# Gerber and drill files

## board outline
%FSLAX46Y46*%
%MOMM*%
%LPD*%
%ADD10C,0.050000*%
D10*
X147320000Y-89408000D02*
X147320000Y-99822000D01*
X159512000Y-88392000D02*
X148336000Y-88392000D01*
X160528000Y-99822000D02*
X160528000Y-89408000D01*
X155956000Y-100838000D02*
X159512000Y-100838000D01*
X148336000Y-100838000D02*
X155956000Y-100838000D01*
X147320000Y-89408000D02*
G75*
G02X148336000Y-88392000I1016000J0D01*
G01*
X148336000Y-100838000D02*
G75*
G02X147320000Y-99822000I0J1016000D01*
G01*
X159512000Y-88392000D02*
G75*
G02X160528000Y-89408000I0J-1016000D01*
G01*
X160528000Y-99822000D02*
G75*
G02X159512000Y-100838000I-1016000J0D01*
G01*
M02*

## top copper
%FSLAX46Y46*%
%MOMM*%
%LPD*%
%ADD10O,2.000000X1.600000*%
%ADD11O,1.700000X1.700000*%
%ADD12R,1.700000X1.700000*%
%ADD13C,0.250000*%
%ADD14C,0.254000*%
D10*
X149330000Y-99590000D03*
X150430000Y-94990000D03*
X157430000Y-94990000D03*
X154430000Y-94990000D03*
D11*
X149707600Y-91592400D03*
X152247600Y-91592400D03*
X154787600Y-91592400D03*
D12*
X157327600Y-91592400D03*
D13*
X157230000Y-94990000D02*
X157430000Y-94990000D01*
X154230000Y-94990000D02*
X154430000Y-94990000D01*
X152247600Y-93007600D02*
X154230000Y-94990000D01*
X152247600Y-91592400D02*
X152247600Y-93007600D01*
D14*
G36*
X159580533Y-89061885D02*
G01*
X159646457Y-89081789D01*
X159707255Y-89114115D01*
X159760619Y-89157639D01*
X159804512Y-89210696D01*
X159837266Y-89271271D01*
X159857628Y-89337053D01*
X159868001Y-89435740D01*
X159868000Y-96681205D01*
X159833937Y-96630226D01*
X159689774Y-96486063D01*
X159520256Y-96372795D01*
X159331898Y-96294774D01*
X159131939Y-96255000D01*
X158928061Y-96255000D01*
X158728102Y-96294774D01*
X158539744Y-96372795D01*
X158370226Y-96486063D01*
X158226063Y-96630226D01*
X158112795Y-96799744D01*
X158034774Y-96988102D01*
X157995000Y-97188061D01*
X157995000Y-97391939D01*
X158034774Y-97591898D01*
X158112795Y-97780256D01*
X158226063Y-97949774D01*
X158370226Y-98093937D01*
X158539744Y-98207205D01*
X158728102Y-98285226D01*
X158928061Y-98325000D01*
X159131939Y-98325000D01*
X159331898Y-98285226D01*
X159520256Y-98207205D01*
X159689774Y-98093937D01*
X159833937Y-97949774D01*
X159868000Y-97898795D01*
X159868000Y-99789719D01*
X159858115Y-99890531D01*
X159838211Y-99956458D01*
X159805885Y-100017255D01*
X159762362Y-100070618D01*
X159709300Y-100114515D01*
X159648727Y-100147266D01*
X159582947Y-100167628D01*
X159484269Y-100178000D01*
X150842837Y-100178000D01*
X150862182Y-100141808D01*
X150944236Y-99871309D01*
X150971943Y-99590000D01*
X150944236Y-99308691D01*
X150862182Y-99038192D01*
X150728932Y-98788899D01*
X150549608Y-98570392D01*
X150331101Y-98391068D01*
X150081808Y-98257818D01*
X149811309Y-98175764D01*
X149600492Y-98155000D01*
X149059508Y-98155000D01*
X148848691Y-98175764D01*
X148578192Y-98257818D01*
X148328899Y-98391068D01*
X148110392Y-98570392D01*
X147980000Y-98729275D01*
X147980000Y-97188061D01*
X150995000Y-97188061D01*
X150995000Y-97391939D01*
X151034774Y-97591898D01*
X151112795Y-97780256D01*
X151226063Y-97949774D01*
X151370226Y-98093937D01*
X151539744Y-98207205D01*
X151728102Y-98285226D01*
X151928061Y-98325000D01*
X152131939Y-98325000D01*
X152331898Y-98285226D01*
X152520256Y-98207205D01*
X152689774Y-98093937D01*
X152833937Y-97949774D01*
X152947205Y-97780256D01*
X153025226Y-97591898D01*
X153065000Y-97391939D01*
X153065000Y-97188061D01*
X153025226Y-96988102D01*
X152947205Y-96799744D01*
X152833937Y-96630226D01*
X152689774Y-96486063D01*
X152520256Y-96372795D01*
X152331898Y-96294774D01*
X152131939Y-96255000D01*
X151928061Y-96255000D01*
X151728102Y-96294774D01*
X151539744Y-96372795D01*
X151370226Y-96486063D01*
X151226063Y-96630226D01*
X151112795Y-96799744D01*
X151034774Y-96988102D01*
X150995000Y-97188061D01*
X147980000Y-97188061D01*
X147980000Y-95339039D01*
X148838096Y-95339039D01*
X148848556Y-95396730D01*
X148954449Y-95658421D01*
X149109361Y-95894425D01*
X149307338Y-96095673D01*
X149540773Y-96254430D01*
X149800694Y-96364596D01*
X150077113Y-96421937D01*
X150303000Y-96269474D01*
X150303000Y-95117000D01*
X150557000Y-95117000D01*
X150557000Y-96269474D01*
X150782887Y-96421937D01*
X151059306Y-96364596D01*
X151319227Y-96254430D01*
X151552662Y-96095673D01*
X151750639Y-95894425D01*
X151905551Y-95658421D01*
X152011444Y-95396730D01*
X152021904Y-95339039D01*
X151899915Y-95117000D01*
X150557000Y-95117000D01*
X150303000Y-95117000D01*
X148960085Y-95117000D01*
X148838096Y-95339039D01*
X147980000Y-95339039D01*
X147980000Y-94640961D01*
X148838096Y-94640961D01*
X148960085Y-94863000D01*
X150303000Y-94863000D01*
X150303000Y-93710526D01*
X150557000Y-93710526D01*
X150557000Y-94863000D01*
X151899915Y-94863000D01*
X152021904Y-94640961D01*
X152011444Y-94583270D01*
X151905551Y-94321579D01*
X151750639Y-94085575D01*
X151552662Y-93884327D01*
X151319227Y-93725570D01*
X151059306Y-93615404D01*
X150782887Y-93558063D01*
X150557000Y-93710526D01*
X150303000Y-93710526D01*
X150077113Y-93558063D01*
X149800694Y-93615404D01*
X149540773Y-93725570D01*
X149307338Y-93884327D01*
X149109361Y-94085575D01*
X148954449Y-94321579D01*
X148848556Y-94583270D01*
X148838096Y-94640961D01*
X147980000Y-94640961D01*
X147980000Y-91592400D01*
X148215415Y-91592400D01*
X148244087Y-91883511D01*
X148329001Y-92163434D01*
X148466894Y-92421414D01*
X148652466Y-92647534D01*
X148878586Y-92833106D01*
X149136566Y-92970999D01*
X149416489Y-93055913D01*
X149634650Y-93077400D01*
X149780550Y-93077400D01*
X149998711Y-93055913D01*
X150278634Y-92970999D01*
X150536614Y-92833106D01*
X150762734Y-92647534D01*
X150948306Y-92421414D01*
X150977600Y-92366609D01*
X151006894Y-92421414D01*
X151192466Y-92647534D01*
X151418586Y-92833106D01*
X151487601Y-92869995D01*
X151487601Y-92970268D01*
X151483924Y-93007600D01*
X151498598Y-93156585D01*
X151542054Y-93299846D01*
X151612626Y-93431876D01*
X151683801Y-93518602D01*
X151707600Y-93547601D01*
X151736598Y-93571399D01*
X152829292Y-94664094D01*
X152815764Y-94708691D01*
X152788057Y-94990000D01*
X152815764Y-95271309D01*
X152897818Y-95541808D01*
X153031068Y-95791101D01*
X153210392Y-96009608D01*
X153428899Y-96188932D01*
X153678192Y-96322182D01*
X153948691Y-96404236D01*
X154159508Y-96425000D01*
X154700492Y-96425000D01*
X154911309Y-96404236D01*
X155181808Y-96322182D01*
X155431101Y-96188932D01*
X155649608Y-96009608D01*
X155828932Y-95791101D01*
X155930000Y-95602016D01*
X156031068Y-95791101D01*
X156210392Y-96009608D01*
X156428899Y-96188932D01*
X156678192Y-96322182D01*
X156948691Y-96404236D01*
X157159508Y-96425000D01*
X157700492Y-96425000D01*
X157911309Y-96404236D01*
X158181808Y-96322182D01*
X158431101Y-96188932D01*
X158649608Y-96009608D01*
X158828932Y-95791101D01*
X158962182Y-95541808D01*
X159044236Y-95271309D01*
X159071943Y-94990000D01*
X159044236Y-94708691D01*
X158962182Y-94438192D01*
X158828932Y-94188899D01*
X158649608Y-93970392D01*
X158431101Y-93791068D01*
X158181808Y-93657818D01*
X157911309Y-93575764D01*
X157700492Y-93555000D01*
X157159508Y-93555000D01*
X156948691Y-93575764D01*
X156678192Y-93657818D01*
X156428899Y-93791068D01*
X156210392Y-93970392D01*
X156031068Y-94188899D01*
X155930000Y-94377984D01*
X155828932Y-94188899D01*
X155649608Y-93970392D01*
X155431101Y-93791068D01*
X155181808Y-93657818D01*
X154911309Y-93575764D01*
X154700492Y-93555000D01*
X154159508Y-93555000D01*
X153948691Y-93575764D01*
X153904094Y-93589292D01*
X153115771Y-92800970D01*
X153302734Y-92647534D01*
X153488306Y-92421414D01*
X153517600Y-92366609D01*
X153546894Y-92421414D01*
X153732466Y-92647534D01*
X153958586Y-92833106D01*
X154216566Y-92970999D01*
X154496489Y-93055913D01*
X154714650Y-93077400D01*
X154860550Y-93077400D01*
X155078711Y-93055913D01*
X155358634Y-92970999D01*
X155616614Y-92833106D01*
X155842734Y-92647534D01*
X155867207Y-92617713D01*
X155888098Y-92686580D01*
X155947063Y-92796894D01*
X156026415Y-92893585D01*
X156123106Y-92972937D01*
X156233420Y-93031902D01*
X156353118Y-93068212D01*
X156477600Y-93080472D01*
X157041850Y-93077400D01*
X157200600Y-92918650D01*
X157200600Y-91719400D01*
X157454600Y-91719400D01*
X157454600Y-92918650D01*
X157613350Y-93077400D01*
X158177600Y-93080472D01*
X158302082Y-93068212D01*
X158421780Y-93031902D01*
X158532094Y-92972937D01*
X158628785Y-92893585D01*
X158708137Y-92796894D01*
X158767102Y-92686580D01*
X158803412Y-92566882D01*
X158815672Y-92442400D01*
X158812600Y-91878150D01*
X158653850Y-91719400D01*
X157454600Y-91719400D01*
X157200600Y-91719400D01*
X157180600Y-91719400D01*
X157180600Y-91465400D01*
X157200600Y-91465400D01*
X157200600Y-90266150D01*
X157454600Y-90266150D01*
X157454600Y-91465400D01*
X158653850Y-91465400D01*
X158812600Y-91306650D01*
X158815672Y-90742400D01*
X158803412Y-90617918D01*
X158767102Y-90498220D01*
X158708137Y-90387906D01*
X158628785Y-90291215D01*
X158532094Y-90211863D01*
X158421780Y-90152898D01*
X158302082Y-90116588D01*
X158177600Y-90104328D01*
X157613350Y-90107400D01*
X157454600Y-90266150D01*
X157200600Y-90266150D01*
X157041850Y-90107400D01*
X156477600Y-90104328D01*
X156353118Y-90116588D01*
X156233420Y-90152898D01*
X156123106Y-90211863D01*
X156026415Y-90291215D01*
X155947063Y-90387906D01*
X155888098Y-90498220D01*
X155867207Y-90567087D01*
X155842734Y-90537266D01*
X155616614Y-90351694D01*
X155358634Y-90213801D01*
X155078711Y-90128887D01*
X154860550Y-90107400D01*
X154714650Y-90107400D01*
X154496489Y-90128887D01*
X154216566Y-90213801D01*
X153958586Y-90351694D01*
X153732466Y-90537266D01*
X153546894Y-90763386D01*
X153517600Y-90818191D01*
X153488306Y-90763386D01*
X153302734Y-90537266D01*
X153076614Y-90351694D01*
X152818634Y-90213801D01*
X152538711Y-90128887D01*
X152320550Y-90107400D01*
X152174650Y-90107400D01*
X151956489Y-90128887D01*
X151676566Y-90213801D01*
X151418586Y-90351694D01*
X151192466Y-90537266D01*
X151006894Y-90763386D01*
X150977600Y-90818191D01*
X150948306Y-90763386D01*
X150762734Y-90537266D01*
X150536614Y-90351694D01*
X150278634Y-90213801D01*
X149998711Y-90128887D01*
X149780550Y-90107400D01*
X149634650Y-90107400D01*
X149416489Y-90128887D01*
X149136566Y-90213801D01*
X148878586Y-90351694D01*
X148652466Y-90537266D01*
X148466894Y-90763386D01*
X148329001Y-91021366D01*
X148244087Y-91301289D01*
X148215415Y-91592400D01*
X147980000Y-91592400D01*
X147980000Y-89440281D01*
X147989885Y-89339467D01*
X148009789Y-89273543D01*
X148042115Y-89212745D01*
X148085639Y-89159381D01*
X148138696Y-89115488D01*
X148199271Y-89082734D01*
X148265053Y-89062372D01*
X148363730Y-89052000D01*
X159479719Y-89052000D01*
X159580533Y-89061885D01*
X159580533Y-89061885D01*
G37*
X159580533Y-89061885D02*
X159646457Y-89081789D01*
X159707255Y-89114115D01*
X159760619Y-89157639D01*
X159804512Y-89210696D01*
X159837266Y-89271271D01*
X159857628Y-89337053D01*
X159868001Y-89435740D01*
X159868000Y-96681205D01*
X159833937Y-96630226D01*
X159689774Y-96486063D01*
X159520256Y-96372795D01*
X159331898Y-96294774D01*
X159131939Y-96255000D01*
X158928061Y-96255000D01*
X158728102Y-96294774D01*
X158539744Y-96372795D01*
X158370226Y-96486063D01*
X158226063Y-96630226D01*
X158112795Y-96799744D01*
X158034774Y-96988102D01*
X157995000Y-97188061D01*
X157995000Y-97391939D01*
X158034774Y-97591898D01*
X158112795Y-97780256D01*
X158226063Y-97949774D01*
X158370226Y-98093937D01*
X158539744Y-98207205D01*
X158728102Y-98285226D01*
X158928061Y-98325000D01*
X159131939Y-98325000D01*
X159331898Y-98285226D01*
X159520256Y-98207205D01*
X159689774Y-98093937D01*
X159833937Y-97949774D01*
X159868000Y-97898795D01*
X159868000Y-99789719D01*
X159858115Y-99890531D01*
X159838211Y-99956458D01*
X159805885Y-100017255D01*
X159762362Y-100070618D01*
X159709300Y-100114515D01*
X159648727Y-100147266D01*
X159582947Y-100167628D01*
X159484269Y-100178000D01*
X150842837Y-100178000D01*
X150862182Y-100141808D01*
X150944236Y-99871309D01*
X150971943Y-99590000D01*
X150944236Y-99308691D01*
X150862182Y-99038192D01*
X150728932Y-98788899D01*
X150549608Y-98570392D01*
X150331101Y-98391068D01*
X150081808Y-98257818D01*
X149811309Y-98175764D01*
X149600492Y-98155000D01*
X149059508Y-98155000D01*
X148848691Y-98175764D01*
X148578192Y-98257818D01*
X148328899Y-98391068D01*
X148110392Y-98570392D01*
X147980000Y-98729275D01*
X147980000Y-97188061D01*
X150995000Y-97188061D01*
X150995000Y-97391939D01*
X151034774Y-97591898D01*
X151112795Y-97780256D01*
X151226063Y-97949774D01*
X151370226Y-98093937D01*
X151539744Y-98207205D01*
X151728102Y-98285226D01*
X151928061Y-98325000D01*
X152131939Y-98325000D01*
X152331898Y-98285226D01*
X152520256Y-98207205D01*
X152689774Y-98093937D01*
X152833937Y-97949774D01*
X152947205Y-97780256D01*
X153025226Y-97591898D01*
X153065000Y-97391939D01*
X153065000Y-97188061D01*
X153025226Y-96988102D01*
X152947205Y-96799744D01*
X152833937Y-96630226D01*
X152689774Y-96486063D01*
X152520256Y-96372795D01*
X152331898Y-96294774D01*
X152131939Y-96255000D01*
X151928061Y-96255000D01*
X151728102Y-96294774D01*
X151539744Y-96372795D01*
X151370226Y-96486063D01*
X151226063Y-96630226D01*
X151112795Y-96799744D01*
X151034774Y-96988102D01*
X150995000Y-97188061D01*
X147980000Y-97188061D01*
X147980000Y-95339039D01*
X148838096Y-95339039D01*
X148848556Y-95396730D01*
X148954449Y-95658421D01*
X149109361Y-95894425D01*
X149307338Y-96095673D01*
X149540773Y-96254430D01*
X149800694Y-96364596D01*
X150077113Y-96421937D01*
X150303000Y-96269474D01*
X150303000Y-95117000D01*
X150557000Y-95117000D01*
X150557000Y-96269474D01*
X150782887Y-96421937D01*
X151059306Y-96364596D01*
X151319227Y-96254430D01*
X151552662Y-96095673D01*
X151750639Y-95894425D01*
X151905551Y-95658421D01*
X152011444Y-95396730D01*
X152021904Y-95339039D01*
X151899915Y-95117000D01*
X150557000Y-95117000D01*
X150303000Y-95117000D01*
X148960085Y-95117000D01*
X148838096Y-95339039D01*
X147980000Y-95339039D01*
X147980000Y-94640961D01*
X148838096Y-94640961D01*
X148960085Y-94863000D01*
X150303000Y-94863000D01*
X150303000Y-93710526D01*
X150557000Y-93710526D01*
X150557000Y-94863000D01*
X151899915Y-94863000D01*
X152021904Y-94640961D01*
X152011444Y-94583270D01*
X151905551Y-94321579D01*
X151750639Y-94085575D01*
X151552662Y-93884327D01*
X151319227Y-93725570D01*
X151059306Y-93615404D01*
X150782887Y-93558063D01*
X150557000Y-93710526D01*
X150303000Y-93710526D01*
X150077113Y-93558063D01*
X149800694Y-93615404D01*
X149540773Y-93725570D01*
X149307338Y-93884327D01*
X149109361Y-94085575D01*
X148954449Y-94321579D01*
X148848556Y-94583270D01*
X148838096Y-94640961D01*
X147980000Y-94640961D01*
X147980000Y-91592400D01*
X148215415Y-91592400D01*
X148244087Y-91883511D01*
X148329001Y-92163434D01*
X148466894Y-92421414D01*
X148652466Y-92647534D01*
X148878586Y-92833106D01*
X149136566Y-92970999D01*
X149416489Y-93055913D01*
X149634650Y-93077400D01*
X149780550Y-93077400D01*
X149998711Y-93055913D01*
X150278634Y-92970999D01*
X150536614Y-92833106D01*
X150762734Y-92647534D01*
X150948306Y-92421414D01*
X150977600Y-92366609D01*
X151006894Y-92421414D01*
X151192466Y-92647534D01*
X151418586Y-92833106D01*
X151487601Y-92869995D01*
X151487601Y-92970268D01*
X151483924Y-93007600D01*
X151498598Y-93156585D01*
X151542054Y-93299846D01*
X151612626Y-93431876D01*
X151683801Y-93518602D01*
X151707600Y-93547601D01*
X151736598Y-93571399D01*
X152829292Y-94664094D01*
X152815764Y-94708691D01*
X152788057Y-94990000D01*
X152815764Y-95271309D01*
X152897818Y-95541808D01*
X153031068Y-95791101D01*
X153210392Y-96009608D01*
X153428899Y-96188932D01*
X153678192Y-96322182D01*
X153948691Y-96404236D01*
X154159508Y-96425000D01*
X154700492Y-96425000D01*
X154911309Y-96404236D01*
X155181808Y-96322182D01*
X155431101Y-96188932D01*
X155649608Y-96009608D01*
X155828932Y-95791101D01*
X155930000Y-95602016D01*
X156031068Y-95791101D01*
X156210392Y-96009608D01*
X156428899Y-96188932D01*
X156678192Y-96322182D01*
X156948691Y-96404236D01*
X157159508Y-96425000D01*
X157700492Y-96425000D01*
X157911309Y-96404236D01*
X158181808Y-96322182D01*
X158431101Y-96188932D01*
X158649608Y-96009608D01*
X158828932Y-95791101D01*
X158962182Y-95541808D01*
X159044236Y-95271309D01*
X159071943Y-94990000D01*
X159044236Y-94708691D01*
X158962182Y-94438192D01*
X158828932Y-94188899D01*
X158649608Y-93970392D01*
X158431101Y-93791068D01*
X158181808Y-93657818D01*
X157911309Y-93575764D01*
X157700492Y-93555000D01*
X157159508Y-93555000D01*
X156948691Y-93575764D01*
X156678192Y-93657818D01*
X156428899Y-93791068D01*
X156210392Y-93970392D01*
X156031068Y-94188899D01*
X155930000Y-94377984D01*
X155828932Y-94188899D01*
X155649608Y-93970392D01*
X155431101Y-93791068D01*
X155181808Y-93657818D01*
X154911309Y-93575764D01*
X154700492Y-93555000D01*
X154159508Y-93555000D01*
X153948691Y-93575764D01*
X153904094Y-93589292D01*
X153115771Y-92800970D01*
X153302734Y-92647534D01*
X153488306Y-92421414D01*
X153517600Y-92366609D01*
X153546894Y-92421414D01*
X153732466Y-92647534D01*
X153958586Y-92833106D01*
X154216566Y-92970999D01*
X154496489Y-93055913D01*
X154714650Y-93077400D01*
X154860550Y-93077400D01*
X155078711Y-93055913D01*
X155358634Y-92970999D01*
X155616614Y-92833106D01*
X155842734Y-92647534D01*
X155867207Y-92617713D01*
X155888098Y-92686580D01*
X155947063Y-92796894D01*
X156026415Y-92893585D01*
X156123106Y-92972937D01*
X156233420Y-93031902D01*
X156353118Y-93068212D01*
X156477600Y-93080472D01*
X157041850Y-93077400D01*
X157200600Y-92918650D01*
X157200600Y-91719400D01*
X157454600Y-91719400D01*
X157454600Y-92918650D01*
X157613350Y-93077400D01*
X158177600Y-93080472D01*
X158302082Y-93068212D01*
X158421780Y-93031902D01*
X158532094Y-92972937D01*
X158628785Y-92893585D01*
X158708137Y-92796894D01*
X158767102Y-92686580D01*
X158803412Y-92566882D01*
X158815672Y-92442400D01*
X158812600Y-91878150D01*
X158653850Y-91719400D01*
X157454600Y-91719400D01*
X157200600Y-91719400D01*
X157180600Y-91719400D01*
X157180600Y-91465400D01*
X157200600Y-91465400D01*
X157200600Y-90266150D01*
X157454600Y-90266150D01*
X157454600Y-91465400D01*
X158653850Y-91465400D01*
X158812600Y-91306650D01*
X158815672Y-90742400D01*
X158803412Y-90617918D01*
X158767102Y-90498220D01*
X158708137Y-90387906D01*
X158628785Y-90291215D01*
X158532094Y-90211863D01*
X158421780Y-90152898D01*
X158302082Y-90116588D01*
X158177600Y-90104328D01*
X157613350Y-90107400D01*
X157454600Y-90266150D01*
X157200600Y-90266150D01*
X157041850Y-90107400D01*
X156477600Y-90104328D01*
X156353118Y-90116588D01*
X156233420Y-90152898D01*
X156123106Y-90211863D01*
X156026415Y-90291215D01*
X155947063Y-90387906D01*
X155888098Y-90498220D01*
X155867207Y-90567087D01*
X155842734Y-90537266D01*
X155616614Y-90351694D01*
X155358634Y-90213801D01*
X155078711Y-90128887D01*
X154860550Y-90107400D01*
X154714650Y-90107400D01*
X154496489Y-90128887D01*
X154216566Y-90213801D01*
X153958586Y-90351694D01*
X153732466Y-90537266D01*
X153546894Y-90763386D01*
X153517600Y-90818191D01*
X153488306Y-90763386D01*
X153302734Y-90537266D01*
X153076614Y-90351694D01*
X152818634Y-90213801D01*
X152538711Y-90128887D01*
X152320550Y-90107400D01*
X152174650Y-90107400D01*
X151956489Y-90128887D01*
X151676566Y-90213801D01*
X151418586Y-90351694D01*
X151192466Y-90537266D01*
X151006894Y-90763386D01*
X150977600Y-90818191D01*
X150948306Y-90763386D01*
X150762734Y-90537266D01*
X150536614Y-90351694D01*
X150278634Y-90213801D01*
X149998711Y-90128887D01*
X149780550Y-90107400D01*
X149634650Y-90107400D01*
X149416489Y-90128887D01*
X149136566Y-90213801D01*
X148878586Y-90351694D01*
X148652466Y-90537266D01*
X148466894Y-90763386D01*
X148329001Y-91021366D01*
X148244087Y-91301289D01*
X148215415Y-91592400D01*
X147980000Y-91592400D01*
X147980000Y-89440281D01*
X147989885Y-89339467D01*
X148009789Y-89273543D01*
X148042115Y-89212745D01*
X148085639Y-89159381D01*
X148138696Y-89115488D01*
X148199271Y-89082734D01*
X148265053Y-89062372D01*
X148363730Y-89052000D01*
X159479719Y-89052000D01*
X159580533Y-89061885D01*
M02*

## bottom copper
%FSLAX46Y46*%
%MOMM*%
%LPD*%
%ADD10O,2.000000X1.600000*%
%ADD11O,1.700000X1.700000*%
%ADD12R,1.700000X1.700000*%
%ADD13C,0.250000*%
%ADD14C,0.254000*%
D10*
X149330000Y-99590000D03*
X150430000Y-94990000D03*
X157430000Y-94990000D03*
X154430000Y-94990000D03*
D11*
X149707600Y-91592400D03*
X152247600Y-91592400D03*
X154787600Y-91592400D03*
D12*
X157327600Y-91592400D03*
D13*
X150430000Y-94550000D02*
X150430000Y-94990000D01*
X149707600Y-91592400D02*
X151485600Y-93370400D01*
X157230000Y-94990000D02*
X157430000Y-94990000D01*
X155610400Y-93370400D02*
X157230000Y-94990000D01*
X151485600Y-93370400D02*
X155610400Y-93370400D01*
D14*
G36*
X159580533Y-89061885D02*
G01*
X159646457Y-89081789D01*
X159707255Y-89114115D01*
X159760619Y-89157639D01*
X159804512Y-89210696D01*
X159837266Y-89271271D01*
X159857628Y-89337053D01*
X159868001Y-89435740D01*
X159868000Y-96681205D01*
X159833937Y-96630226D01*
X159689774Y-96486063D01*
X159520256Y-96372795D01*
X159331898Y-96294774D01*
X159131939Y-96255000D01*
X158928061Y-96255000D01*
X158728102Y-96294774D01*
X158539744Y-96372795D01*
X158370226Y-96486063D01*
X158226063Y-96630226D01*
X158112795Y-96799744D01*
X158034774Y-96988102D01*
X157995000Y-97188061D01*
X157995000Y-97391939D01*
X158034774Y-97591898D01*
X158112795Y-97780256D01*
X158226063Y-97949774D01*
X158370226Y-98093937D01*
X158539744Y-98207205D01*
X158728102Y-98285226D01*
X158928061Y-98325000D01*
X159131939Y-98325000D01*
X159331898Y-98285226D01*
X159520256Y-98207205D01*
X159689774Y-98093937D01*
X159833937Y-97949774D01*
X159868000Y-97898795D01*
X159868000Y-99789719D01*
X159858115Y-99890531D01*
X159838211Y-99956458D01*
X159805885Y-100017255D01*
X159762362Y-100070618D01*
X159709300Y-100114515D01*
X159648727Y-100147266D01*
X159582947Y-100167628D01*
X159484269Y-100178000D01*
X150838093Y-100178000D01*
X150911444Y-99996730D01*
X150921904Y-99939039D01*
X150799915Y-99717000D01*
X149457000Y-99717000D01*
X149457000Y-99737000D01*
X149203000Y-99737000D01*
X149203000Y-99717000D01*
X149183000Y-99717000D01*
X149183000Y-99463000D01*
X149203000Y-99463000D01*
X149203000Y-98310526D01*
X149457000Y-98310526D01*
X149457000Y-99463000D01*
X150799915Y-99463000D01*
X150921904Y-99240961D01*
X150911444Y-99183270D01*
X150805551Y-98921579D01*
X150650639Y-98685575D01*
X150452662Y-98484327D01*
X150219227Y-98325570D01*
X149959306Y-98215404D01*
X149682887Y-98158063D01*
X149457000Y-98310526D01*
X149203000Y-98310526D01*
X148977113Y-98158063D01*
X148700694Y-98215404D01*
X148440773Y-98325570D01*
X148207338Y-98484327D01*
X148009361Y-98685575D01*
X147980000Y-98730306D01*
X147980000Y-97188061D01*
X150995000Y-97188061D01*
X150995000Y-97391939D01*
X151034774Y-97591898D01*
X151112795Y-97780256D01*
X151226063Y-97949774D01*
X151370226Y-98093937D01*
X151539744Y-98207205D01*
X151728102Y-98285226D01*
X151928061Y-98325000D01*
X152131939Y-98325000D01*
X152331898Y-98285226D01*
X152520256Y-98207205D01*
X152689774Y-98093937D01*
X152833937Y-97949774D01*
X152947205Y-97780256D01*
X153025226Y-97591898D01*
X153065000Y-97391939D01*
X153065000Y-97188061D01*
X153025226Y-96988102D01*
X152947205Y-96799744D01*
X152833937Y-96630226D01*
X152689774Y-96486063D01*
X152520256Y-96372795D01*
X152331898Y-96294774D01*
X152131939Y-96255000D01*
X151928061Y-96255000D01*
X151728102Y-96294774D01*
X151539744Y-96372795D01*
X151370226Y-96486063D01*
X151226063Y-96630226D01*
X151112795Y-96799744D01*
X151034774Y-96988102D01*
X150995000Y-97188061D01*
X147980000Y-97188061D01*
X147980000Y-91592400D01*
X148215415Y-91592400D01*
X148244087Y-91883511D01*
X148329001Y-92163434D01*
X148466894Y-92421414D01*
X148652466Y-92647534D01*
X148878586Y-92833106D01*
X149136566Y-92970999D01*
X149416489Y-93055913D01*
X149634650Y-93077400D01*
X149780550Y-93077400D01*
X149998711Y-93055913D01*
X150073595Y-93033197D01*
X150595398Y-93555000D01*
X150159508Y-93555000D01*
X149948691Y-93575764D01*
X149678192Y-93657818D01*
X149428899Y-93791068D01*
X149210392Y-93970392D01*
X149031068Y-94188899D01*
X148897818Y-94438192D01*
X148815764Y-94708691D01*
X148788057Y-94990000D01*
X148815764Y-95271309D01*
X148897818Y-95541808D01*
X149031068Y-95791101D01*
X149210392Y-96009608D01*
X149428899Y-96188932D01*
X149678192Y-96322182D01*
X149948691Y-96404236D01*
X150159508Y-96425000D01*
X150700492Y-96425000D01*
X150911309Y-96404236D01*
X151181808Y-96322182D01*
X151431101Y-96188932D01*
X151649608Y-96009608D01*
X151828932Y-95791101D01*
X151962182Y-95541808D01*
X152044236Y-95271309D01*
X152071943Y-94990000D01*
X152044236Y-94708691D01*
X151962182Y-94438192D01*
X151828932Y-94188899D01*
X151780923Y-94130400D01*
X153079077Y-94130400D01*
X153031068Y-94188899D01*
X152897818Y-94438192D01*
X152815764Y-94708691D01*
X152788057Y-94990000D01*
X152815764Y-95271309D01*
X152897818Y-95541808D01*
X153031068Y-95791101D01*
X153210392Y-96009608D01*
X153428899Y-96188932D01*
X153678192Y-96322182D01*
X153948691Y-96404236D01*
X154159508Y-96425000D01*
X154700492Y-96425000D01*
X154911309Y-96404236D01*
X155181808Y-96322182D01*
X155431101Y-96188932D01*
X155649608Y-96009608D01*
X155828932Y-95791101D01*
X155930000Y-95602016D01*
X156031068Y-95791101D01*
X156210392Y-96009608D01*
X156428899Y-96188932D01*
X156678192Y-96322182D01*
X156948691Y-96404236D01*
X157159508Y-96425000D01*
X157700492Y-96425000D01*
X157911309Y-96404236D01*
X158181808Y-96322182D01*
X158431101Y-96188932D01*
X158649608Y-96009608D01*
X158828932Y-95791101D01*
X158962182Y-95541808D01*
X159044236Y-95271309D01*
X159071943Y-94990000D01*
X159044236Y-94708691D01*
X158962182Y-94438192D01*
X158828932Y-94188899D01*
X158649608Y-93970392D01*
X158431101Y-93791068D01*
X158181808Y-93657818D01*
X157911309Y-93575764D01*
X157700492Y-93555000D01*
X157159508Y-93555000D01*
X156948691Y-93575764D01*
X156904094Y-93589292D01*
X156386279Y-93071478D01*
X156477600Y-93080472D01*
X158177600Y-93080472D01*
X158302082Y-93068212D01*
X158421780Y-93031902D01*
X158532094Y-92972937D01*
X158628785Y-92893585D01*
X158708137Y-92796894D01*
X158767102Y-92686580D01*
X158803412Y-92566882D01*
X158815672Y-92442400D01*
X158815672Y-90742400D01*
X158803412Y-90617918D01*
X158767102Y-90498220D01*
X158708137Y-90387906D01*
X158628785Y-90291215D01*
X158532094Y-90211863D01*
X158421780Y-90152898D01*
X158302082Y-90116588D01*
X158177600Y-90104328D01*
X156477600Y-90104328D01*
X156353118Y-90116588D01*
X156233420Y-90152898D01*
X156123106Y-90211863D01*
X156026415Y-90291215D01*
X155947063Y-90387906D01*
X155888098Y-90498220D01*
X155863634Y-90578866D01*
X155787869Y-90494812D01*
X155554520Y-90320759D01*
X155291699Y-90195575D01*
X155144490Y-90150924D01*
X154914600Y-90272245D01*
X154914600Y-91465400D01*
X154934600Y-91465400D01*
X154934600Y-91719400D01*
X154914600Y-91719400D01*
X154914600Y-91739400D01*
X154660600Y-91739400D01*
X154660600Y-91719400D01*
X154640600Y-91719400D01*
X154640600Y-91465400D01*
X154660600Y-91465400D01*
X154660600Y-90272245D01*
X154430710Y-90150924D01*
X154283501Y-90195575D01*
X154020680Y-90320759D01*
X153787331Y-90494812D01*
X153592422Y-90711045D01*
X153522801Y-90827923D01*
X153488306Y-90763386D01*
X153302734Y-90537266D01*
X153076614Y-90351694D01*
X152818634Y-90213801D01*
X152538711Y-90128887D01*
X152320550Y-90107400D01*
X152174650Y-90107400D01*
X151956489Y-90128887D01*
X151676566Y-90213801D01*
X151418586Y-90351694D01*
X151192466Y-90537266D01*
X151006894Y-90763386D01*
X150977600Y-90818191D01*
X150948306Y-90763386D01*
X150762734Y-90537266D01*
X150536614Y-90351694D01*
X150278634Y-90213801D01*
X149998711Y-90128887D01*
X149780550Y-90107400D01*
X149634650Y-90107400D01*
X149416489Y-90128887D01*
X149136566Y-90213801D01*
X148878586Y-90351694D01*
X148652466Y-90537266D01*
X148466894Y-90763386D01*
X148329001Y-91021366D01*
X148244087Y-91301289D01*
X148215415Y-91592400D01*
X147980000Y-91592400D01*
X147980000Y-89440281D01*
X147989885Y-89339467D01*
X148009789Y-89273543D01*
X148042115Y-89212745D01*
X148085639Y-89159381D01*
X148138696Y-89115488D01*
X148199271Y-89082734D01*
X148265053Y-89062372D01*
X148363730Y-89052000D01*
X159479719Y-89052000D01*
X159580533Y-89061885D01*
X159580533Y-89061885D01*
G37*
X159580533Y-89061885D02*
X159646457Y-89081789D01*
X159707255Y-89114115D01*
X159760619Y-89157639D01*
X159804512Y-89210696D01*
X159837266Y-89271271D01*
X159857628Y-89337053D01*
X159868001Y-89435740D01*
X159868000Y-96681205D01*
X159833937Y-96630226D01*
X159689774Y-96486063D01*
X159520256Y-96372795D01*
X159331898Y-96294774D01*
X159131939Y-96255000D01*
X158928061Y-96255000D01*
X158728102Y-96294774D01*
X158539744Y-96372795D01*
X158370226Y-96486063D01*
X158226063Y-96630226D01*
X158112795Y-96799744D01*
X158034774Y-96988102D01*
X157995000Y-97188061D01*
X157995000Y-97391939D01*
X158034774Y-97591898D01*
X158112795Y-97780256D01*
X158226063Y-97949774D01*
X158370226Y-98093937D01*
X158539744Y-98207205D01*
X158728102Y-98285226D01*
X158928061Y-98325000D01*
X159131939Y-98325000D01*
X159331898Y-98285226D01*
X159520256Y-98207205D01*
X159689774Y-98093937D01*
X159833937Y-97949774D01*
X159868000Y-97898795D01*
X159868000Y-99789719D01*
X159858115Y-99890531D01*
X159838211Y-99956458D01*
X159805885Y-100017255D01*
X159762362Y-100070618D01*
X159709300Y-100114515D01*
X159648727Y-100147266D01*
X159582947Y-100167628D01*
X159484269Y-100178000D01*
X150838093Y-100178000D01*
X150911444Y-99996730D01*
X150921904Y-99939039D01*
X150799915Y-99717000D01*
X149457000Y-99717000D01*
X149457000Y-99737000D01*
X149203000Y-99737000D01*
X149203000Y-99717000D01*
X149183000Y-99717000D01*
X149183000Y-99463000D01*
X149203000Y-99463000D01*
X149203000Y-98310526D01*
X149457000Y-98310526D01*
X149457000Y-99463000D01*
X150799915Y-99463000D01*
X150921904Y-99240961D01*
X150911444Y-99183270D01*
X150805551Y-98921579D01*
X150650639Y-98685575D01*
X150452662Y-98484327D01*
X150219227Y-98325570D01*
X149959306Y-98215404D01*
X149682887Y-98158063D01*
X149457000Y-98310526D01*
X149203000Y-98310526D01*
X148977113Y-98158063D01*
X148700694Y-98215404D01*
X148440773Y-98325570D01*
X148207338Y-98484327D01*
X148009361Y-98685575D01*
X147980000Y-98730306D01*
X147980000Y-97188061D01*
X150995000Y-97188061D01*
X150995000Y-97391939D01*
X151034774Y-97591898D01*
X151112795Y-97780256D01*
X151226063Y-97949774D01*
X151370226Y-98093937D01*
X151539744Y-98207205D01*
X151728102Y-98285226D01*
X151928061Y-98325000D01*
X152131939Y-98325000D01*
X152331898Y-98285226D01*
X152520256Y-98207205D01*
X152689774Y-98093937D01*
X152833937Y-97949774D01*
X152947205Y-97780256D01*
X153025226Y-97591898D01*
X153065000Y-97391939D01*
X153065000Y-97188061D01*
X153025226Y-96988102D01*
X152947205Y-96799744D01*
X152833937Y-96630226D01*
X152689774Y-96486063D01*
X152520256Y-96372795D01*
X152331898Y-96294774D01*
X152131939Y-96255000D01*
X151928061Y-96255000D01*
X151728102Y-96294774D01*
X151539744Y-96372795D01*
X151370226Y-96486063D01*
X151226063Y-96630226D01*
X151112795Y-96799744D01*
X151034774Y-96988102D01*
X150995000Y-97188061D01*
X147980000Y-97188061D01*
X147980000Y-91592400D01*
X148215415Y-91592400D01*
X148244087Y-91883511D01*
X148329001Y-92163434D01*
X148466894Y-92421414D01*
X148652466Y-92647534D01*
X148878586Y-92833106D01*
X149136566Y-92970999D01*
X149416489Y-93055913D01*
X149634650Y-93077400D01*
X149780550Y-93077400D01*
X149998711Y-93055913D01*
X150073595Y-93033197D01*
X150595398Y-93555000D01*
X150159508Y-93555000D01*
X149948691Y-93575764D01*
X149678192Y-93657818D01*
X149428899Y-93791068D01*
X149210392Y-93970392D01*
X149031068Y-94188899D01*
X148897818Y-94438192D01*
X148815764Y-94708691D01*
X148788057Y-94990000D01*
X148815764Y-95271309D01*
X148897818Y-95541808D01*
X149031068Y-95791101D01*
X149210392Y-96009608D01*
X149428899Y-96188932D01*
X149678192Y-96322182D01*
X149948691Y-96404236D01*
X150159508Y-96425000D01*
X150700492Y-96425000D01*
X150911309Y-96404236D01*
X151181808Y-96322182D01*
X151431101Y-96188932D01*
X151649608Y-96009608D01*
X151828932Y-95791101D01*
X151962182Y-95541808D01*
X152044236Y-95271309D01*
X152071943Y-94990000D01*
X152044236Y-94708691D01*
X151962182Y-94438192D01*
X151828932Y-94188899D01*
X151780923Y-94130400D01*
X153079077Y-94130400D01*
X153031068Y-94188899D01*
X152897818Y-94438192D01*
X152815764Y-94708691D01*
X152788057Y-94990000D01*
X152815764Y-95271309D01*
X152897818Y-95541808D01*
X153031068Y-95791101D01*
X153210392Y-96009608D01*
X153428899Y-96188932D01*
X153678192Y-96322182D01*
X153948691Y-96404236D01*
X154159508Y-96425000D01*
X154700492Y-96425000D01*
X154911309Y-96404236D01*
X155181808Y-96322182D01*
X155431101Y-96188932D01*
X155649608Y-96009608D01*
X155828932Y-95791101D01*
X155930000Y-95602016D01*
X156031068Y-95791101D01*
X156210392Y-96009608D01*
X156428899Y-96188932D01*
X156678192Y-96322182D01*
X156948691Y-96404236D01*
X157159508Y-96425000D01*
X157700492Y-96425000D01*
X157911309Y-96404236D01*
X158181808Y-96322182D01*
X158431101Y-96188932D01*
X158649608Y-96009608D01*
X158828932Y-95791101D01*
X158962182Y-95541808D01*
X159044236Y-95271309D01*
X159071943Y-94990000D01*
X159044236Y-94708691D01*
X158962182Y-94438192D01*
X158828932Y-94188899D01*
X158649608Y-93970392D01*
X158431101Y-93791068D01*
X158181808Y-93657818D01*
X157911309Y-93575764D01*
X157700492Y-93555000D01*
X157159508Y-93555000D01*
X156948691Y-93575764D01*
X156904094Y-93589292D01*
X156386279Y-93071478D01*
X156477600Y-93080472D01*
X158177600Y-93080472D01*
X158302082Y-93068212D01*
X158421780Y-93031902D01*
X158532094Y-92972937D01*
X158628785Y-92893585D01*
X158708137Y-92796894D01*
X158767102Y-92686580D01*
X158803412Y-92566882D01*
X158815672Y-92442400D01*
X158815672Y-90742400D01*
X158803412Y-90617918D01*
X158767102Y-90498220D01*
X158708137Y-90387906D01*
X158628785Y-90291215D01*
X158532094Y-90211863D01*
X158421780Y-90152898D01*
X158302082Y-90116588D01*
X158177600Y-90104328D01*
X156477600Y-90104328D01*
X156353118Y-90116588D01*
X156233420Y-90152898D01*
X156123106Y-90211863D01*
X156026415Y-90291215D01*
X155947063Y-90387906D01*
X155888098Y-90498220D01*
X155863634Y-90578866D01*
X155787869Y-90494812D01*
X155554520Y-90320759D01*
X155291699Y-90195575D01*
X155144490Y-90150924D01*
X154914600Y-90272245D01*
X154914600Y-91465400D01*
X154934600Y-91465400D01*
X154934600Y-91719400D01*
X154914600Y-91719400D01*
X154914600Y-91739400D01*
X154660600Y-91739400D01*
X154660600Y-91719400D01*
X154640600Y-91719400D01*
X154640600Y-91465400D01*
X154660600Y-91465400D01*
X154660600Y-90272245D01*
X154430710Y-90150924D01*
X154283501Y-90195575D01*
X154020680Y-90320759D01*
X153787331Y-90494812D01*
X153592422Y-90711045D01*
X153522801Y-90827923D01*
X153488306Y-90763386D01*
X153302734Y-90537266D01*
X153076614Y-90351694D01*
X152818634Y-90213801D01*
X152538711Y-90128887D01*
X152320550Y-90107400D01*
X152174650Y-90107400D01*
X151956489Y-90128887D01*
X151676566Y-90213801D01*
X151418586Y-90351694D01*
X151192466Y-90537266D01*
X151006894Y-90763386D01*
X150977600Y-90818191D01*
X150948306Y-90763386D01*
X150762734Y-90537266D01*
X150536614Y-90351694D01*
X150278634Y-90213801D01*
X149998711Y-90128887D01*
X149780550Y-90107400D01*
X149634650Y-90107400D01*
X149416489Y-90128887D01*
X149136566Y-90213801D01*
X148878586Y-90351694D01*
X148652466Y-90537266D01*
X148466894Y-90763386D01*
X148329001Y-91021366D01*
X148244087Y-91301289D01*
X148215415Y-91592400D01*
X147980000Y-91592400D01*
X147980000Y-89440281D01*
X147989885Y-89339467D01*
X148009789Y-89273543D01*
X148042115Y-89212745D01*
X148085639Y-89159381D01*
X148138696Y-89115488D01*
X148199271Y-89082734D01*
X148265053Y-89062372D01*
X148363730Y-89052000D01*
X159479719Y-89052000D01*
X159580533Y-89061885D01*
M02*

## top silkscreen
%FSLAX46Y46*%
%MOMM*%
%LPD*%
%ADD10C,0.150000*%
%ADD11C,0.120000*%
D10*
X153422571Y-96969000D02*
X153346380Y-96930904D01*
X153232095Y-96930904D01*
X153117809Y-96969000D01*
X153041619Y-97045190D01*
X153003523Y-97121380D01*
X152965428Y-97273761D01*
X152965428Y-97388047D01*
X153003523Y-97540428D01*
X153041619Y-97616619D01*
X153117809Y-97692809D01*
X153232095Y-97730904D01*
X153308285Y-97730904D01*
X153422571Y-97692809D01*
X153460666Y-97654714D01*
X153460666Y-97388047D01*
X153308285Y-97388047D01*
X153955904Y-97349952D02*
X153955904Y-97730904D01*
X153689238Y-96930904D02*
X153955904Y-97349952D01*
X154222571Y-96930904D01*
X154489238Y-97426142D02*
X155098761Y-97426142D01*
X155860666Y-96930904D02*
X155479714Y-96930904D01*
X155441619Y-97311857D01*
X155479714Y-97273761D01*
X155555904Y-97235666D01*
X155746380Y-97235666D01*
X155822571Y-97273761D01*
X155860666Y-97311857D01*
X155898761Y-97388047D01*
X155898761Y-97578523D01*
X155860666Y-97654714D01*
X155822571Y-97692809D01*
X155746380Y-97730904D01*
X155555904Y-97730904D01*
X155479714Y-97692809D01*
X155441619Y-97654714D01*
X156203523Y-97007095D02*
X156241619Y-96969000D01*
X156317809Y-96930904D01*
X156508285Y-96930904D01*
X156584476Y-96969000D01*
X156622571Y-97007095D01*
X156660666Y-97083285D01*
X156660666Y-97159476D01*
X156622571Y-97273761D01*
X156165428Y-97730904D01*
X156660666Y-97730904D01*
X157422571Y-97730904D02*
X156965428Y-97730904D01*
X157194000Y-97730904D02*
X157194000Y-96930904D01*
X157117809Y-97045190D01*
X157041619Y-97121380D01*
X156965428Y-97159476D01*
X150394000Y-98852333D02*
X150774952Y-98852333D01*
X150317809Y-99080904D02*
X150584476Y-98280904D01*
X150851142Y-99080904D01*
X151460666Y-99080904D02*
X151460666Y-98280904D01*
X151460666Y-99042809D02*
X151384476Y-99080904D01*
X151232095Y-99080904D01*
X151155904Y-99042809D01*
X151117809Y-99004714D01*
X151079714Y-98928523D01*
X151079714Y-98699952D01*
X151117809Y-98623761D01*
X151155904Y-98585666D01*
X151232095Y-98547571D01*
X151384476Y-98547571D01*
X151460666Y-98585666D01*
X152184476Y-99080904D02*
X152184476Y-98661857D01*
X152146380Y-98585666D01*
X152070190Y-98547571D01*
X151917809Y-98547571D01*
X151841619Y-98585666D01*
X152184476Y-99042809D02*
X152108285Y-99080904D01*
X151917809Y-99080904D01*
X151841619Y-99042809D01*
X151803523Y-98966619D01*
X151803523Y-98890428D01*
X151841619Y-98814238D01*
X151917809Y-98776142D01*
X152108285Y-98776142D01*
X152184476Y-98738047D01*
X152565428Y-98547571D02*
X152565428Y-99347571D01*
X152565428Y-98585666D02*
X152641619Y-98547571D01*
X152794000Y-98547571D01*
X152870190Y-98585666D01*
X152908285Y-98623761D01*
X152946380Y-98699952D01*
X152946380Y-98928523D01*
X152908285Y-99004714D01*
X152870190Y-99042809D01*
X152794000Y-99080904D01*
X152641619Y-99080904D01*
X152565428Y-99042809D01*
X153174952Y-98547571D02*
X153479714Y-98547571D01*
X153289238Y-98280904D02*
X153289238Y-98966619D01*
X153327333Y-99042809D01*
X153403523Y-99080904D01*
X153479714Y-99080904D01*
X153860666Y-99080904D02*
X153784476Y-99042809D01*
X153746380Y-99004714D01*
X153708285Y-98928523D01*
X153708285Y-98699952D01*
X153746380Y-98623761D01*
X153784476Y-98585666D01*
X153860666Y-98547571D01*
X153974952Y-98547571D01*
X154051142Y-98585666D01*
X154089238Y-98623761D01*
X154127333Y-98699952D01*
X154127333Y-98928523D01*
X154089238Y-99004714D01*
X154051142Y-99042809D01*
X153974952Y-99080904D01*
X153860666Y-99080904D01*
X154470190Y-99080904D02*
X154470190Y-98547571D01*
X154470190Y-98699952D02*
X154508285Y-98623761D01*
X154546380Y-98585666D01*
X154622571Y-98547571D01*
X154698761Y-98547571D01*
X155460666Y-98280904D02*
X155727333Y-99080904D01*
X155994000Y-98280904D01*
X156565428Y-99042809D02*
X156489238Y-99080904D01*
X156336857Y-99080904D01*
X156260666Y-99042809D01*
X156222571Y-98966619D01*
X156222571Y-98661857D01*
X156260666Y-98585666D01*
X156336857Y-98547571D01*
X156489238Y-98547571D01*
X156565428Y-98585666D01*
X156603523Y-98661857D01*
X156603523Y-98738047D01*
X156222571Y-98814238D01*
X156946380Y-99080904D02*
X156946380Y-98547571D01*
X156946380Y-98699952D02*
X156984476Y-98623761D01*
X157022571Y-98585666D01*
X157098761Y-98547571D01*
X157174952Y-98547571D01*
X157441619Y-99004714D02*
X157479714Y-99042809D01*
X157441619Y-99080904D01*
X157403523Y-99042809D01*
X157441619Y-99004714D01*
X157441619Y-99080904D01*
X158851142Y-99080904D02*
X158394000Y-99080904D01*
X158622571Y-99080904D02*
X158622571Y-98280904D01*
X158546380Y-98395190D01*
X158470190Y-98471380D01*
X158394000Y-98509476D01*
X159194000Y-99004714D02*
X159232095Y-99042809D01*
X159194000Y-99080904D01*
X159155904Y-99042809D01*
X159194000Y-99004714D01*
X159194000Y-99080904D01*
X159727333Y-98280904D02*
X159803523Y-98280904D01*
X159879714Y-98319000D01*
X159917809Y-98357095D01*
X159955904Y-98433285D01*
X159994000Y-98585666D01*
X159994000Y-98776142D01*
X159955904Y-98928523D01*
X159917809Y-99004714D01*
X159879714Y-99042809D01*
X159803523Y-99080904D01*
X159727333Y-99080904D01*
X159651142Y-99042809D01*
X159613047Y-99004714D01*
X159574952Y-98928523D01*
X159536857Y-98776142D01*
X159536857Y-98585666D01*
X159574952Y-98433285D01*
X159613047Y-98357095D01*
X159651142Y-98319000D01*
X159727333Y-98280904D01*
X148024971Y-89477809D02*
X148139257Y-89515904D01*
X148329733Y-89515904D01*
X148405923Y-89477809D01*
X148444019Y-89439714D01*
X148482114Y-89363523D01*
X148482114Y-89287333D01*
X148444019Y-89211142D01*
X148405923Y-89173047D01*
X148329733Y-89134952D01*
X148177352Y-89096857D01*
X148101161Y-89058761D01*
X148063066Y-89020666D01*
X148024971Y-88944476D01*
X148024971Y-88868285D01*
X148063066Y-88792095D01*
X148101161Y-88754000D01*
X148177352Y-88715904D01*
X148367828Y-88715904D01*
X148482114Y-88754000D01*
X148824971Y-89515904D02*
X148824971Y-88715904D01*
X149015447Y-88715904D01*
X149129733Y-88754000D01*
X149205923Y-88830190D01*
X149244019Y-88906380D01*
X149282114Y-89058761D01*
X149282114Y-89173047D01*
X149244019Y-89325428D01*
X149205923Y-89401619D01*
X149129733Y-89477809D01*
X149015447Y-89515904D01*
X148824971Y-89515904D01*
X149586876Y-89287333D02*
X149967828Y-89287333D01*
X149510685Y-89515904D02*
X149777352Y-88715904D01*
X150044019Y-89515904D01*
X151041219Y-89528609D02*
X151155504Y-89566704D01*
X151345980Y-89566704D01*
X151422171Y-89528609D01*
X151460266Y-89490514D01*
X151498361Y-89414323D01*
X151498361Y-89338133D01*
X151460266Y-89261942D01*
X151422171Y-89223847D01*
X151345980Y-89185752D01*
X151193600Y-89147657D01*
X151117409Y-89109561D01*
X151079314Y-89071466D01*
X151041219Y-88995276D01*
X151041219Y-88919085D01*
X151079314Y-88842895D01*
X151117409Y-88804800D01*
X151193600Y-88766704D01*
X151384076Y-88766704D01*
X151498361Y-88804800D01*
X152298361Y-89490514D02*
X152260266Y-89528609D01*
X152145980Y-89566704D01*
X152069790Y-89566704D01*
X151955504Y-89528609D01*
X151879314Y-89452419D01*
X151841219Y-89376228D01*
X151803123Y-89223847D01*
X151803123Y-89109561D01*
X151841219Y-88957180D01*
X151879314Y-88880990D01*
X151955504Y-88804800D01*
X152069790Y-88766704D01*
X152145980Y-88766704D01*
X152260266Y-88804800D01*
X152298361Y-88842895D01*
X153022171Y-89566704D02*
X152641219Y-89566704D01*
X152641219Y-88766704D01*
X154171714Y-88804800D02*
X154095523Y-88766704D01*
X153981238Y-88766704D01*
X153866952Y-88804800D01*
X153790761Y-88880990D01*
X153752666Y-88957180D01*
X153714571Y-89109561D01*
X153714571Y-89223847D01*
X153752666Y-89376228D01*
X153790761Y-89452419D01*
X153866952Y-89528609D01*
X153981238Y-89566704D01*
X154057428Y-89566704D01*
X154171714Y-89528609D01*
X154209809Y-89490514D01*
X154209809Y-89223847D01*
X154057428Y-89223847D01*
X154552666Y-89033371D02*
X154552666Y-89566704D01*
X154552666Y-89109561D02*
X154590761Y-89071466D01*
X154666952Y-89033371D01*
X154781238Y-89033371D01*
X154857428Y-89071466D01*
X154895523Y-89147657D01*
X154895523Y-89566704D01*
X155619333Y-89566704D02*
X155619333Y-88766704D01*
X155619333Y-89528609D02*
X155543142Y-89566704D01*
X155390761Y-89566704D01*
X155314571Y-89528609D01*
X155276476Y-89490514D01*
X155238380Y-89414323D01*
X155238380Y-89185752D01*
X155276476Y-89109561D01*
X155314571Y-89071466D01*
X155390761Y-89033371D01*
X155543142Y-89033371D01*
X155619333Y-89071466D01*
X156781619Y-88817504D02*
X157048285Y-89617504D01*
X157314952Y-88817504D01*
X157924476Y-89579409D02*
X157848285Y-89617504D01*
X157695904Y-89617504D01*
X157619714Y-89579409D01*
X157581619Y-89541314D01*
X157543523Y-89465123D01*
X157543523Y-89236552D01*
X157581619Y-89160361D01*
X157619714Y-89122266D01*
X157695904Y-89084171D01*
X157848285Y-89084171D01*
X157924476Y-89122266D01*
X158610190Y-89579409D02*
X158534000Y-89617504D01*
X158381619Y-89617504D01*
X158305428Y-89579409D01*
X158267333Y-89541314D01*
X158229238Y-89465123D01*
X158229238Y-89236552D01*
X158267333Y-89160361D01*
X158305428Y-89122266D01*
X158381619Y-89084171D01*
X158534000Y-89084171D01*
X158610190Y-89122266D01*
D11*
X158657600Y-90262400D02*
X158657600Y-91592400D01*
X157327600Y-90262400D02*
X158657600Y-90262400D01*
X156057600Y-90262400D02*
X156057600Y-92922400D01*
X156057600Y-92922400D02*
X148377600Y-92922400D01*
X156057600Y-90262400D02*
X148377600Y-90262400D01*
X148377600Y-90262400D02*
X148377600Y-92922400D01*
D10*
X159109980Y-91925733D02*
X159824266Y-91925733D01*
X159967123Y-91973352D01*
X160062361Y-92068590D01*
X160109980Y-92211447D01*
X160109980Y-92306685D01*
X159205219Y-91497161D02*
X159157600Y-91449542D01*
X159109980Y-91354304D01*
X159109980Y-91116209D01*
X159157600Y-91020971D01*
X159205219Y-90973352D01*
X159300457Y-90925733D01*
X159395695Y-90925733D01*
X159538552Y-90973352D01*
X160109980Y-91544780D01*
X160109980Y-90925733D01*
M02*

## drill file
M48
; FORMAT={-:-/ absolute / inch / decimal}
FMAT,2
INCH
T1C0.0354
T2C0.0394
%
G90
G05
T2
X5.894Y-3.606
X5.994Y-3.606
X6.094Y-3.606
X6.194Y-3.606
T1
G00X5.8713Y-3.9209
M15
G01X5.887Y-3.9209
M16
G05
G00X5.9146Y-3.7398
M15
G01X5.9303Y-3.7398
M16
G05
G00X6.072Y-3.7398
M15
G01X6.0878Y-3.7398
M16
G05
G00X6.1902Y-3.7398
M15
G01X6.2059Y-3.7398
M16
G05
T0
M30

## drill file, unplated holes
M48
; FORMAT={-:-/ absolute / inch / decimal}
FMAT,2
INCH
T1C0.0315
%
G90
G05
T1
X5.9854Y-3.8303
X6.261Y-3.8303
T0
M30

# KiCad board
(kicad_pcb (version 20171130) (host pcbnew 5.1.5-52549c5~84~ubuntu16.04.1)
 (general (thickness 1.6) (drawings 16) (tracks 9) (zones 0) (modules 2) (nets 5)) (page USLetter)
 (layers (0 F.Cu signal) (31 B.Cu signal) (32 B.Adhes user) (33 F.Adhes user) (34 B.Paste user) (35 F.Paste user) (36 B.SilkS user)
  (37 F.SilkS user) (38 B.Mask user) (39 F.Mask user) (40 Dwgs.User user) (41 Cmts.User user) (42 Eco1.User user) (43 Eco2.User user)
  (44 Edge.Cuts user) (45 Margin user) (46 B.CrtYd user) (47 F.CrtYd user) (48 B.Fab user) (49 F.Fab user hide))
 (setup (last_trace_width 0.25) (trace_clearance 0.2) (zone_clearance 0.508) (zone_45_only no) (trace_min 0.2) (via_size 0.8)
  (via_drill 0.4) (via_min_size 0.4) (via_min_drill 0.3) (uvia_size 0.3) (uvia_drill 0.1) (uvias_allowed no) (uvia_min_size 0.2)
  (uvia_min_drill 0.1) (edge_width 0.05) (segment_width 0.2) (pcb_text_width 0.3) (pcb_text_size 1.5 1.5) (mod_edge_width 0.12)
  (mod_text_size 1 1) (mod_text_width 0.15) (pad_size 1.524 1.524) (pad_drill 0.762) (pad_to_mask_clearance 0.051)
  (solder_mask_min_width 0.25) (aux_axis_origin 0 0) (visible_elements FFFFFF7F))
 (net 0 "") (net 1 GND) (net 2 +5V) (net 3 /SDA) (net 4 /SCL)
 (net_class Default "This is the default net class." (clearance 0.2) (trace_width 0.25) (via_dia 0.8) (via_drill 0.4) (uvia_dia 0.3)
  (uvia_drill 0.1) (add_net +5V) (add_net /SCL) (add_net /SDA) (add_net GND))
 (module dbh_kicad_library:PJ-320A (layer B.Cu) (at 157.48 95.25 180)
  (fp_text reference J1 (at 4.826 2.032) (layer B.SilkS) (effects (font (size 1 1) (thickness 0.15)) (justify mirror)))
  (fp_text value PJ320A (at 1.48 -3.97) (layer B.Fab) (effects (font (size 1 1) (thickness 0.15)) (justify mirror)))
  (pad 5 thru_hole oval (at 8.15 -4.34 90) (size 1.6 2) (drill oval 0.9 1.3) (layers *.Cu *.Mask) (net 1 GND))
  (pad 4 thru_hole oval (at 7.05 0.26 90) (size 1.6 2) (drill oval 0.9 1.3) (layers *.Cu *.Mask) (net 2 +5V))
  (pad 2 thru_hole oval (at 0.05 0.26 90) (size 1.6 2) (drill oval 0.9 1.3) (layers *.Cu *.Mask) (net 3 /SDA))
  (pad "" np_thru_hole circle (at 5.45 -2.04 90) (size 0.8 0.8) (drill 0.8) (layers *.Cu *.Mask))
  (pad "" np_thru_hole circle (at -1.55 -2.04 90) (size 0.8 0.8) (drill 0.8) (layers *.Cu *.Mask))
  (pad 3 thru_hole oval (at 3.05 0.26 90) (size 1.6 2) (drill oval 0.9 1.3) (layers *.Cu *.Mask) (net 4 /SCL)))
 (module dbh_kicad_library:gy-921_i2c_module (layer F.Cu) (at 157.3276 91.5924 270)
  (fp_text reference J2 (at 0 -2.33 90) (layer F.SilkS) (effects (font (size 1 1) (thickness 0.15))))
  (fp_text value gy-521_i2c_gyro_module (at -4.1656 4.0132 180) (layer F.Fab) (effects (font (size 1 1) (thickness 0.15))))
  (fp_line (start -1.33 -1.33) (end 0 -1.33) (layer F.SilkS) (width 0.12))
  (fp_line (start -1.33 0) (end -1.33 -1.33) (layer F.SilkS) (width 0.12))
  (fp_line (start -1.33 1.27) (end 1.33 1.27) (layer F.SilkS) (width 0.12))
  (fp_line (start 1.33 1.27) (end 1.33 8.95) (layer F.SilkS) (width 0.12))
  (fp_line (start -1.33 1.27) (end -1.33 8.95) (layer F.SilkS) (width 0.12))
  (fp_line (start -1.33 8.95) (end 1.33 8.95) (layer F.SilkS) (width 0.12))
  (pad 4 thru_hole oval (at 0 7.62 270) (size 1.7 1.7) (drill 1) (layers *.Cu *.Mask) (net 3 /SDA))
  (pad 3 thru_hole oval (at 0 5.08 270) (size 1.7 1.7) (drill 1) (layers *.Cu *.Mask) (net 4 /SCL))
  (pad 2 thru_hole oval (at 0 2.54 270) (size 1.7 1.7) (drill 1) (layers *.Cu *.Mask) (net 1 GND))
  (pad 1 thru_hole rect (at 0 0 270) (size 1.7 1.7) (drill 1) (layers *.Cu *.Mask) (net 2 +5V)))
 (gr_line (start 147.32 89.408) (end 147.32 99.822) (layer Edge.Cuts) (width 0.05))
 (gr_line (start 159.512 88.392) (end 148.336 88.392) (layer Edge.Cuts) (width 0.05))
 (gr_line (start 160.528 99.822) (end 160.528 89.408) (layer Edge.Cuts) (width 0.05))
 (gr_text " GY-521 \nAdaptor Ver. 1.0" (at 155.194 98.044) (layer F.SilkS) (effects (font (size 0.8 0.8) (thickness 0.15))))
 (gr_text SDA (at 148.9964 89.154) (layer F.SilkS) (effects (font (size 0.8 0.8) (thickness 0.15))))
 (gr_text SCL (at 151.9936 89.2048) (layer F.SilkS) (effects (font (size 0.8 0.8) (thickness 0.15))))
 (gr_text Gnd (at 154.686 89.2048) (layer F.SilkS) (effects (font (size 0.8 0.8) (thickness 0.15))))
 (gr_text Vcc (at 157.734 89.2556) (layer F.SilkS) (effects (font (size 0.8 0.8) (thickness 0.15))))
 (gr_line (start 155.956 100.838) (end 159.512 100.838) (layer Edge.Cuts) (width 0.05))
 (gr_line (start 148.336 100.838) (end 155.956 100.838) (layer Edge.Cuts) (width 0.05))
 (gr_arc (start 148.336 89.408) (end 148.336 88.392) (angle -90) (layer Edge.Cuts) (width 0.05))
 (gr_arc (start 148.336 99.822) (end 147.32 99.822) (angle -90) (layer Edge.Cuts) (width 0.05))
 (gr_arc (start 159.512 89.408) (end 160.528 89.408) (angle -90) (layer Edge.Cuts) (width 0.05))
 (gr_arc (start 159.512 99.822) (end 159.512 100.838) (angle -90) (layer Edge.Cuts) (width 0.05))
 (segment (start 150.43 94.55) (end 150.43 94.99) (width 0.25) (layer B.Cu) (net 2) (status 30))
 (segment (start 157.23 94.99) (end 157.43 94.99) (width 0.25) (layer F.Cu) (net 3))
 (segment (start 149.7076 91.5924) (end 151.4856 93.3704) (width 0.25) (layer B.Cu) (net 3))
 (segment (start 157.23 94.99) (end 157.43 94.99) (width 0.25) (layer B.Cu) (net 3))
 (segment (start 155.6104 93.3704) (end 157.23 94.99) (width 0.25) (layer B.Cu) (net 3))
 (segment (start 151.4856 93.3704) (end 155.6104 93.3704) (width 0.25) (layer B.Cu) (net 3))
 (segment (start 154.23 94.99) (end 154.43 94.99) (width 0.25) (layer F.Cu) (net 4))
 (segment (start 152.2476 93.0076) (end 154.23 94.99) (width 0.25) (layer F.Cu) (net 4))
 (segment (start 152.2476 91.5924) (end 152.2476 93.0076) (width 0.25) (layer F.Cu) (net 4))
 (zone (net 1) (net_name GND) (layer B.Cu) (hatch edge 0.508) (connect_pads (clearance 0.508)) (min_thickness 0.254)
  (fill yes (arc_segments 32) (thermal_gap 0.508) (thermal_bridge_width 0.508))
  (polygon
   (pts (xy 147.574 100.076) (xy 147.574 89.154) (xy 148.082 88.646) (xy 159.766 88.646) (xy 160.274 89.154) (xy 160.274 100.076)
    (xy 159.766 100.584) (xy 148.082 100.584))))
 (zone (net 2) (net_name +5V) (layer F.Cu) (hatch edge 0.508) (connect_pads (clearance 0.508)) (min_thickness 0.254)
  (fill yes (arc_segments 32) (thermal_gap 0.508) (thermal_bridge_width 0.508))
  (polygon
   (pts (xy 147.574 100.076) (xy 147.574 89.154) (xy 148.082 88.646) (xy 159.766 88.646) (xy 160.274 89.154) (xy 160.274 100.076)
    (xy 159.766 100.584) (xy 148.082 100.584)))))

